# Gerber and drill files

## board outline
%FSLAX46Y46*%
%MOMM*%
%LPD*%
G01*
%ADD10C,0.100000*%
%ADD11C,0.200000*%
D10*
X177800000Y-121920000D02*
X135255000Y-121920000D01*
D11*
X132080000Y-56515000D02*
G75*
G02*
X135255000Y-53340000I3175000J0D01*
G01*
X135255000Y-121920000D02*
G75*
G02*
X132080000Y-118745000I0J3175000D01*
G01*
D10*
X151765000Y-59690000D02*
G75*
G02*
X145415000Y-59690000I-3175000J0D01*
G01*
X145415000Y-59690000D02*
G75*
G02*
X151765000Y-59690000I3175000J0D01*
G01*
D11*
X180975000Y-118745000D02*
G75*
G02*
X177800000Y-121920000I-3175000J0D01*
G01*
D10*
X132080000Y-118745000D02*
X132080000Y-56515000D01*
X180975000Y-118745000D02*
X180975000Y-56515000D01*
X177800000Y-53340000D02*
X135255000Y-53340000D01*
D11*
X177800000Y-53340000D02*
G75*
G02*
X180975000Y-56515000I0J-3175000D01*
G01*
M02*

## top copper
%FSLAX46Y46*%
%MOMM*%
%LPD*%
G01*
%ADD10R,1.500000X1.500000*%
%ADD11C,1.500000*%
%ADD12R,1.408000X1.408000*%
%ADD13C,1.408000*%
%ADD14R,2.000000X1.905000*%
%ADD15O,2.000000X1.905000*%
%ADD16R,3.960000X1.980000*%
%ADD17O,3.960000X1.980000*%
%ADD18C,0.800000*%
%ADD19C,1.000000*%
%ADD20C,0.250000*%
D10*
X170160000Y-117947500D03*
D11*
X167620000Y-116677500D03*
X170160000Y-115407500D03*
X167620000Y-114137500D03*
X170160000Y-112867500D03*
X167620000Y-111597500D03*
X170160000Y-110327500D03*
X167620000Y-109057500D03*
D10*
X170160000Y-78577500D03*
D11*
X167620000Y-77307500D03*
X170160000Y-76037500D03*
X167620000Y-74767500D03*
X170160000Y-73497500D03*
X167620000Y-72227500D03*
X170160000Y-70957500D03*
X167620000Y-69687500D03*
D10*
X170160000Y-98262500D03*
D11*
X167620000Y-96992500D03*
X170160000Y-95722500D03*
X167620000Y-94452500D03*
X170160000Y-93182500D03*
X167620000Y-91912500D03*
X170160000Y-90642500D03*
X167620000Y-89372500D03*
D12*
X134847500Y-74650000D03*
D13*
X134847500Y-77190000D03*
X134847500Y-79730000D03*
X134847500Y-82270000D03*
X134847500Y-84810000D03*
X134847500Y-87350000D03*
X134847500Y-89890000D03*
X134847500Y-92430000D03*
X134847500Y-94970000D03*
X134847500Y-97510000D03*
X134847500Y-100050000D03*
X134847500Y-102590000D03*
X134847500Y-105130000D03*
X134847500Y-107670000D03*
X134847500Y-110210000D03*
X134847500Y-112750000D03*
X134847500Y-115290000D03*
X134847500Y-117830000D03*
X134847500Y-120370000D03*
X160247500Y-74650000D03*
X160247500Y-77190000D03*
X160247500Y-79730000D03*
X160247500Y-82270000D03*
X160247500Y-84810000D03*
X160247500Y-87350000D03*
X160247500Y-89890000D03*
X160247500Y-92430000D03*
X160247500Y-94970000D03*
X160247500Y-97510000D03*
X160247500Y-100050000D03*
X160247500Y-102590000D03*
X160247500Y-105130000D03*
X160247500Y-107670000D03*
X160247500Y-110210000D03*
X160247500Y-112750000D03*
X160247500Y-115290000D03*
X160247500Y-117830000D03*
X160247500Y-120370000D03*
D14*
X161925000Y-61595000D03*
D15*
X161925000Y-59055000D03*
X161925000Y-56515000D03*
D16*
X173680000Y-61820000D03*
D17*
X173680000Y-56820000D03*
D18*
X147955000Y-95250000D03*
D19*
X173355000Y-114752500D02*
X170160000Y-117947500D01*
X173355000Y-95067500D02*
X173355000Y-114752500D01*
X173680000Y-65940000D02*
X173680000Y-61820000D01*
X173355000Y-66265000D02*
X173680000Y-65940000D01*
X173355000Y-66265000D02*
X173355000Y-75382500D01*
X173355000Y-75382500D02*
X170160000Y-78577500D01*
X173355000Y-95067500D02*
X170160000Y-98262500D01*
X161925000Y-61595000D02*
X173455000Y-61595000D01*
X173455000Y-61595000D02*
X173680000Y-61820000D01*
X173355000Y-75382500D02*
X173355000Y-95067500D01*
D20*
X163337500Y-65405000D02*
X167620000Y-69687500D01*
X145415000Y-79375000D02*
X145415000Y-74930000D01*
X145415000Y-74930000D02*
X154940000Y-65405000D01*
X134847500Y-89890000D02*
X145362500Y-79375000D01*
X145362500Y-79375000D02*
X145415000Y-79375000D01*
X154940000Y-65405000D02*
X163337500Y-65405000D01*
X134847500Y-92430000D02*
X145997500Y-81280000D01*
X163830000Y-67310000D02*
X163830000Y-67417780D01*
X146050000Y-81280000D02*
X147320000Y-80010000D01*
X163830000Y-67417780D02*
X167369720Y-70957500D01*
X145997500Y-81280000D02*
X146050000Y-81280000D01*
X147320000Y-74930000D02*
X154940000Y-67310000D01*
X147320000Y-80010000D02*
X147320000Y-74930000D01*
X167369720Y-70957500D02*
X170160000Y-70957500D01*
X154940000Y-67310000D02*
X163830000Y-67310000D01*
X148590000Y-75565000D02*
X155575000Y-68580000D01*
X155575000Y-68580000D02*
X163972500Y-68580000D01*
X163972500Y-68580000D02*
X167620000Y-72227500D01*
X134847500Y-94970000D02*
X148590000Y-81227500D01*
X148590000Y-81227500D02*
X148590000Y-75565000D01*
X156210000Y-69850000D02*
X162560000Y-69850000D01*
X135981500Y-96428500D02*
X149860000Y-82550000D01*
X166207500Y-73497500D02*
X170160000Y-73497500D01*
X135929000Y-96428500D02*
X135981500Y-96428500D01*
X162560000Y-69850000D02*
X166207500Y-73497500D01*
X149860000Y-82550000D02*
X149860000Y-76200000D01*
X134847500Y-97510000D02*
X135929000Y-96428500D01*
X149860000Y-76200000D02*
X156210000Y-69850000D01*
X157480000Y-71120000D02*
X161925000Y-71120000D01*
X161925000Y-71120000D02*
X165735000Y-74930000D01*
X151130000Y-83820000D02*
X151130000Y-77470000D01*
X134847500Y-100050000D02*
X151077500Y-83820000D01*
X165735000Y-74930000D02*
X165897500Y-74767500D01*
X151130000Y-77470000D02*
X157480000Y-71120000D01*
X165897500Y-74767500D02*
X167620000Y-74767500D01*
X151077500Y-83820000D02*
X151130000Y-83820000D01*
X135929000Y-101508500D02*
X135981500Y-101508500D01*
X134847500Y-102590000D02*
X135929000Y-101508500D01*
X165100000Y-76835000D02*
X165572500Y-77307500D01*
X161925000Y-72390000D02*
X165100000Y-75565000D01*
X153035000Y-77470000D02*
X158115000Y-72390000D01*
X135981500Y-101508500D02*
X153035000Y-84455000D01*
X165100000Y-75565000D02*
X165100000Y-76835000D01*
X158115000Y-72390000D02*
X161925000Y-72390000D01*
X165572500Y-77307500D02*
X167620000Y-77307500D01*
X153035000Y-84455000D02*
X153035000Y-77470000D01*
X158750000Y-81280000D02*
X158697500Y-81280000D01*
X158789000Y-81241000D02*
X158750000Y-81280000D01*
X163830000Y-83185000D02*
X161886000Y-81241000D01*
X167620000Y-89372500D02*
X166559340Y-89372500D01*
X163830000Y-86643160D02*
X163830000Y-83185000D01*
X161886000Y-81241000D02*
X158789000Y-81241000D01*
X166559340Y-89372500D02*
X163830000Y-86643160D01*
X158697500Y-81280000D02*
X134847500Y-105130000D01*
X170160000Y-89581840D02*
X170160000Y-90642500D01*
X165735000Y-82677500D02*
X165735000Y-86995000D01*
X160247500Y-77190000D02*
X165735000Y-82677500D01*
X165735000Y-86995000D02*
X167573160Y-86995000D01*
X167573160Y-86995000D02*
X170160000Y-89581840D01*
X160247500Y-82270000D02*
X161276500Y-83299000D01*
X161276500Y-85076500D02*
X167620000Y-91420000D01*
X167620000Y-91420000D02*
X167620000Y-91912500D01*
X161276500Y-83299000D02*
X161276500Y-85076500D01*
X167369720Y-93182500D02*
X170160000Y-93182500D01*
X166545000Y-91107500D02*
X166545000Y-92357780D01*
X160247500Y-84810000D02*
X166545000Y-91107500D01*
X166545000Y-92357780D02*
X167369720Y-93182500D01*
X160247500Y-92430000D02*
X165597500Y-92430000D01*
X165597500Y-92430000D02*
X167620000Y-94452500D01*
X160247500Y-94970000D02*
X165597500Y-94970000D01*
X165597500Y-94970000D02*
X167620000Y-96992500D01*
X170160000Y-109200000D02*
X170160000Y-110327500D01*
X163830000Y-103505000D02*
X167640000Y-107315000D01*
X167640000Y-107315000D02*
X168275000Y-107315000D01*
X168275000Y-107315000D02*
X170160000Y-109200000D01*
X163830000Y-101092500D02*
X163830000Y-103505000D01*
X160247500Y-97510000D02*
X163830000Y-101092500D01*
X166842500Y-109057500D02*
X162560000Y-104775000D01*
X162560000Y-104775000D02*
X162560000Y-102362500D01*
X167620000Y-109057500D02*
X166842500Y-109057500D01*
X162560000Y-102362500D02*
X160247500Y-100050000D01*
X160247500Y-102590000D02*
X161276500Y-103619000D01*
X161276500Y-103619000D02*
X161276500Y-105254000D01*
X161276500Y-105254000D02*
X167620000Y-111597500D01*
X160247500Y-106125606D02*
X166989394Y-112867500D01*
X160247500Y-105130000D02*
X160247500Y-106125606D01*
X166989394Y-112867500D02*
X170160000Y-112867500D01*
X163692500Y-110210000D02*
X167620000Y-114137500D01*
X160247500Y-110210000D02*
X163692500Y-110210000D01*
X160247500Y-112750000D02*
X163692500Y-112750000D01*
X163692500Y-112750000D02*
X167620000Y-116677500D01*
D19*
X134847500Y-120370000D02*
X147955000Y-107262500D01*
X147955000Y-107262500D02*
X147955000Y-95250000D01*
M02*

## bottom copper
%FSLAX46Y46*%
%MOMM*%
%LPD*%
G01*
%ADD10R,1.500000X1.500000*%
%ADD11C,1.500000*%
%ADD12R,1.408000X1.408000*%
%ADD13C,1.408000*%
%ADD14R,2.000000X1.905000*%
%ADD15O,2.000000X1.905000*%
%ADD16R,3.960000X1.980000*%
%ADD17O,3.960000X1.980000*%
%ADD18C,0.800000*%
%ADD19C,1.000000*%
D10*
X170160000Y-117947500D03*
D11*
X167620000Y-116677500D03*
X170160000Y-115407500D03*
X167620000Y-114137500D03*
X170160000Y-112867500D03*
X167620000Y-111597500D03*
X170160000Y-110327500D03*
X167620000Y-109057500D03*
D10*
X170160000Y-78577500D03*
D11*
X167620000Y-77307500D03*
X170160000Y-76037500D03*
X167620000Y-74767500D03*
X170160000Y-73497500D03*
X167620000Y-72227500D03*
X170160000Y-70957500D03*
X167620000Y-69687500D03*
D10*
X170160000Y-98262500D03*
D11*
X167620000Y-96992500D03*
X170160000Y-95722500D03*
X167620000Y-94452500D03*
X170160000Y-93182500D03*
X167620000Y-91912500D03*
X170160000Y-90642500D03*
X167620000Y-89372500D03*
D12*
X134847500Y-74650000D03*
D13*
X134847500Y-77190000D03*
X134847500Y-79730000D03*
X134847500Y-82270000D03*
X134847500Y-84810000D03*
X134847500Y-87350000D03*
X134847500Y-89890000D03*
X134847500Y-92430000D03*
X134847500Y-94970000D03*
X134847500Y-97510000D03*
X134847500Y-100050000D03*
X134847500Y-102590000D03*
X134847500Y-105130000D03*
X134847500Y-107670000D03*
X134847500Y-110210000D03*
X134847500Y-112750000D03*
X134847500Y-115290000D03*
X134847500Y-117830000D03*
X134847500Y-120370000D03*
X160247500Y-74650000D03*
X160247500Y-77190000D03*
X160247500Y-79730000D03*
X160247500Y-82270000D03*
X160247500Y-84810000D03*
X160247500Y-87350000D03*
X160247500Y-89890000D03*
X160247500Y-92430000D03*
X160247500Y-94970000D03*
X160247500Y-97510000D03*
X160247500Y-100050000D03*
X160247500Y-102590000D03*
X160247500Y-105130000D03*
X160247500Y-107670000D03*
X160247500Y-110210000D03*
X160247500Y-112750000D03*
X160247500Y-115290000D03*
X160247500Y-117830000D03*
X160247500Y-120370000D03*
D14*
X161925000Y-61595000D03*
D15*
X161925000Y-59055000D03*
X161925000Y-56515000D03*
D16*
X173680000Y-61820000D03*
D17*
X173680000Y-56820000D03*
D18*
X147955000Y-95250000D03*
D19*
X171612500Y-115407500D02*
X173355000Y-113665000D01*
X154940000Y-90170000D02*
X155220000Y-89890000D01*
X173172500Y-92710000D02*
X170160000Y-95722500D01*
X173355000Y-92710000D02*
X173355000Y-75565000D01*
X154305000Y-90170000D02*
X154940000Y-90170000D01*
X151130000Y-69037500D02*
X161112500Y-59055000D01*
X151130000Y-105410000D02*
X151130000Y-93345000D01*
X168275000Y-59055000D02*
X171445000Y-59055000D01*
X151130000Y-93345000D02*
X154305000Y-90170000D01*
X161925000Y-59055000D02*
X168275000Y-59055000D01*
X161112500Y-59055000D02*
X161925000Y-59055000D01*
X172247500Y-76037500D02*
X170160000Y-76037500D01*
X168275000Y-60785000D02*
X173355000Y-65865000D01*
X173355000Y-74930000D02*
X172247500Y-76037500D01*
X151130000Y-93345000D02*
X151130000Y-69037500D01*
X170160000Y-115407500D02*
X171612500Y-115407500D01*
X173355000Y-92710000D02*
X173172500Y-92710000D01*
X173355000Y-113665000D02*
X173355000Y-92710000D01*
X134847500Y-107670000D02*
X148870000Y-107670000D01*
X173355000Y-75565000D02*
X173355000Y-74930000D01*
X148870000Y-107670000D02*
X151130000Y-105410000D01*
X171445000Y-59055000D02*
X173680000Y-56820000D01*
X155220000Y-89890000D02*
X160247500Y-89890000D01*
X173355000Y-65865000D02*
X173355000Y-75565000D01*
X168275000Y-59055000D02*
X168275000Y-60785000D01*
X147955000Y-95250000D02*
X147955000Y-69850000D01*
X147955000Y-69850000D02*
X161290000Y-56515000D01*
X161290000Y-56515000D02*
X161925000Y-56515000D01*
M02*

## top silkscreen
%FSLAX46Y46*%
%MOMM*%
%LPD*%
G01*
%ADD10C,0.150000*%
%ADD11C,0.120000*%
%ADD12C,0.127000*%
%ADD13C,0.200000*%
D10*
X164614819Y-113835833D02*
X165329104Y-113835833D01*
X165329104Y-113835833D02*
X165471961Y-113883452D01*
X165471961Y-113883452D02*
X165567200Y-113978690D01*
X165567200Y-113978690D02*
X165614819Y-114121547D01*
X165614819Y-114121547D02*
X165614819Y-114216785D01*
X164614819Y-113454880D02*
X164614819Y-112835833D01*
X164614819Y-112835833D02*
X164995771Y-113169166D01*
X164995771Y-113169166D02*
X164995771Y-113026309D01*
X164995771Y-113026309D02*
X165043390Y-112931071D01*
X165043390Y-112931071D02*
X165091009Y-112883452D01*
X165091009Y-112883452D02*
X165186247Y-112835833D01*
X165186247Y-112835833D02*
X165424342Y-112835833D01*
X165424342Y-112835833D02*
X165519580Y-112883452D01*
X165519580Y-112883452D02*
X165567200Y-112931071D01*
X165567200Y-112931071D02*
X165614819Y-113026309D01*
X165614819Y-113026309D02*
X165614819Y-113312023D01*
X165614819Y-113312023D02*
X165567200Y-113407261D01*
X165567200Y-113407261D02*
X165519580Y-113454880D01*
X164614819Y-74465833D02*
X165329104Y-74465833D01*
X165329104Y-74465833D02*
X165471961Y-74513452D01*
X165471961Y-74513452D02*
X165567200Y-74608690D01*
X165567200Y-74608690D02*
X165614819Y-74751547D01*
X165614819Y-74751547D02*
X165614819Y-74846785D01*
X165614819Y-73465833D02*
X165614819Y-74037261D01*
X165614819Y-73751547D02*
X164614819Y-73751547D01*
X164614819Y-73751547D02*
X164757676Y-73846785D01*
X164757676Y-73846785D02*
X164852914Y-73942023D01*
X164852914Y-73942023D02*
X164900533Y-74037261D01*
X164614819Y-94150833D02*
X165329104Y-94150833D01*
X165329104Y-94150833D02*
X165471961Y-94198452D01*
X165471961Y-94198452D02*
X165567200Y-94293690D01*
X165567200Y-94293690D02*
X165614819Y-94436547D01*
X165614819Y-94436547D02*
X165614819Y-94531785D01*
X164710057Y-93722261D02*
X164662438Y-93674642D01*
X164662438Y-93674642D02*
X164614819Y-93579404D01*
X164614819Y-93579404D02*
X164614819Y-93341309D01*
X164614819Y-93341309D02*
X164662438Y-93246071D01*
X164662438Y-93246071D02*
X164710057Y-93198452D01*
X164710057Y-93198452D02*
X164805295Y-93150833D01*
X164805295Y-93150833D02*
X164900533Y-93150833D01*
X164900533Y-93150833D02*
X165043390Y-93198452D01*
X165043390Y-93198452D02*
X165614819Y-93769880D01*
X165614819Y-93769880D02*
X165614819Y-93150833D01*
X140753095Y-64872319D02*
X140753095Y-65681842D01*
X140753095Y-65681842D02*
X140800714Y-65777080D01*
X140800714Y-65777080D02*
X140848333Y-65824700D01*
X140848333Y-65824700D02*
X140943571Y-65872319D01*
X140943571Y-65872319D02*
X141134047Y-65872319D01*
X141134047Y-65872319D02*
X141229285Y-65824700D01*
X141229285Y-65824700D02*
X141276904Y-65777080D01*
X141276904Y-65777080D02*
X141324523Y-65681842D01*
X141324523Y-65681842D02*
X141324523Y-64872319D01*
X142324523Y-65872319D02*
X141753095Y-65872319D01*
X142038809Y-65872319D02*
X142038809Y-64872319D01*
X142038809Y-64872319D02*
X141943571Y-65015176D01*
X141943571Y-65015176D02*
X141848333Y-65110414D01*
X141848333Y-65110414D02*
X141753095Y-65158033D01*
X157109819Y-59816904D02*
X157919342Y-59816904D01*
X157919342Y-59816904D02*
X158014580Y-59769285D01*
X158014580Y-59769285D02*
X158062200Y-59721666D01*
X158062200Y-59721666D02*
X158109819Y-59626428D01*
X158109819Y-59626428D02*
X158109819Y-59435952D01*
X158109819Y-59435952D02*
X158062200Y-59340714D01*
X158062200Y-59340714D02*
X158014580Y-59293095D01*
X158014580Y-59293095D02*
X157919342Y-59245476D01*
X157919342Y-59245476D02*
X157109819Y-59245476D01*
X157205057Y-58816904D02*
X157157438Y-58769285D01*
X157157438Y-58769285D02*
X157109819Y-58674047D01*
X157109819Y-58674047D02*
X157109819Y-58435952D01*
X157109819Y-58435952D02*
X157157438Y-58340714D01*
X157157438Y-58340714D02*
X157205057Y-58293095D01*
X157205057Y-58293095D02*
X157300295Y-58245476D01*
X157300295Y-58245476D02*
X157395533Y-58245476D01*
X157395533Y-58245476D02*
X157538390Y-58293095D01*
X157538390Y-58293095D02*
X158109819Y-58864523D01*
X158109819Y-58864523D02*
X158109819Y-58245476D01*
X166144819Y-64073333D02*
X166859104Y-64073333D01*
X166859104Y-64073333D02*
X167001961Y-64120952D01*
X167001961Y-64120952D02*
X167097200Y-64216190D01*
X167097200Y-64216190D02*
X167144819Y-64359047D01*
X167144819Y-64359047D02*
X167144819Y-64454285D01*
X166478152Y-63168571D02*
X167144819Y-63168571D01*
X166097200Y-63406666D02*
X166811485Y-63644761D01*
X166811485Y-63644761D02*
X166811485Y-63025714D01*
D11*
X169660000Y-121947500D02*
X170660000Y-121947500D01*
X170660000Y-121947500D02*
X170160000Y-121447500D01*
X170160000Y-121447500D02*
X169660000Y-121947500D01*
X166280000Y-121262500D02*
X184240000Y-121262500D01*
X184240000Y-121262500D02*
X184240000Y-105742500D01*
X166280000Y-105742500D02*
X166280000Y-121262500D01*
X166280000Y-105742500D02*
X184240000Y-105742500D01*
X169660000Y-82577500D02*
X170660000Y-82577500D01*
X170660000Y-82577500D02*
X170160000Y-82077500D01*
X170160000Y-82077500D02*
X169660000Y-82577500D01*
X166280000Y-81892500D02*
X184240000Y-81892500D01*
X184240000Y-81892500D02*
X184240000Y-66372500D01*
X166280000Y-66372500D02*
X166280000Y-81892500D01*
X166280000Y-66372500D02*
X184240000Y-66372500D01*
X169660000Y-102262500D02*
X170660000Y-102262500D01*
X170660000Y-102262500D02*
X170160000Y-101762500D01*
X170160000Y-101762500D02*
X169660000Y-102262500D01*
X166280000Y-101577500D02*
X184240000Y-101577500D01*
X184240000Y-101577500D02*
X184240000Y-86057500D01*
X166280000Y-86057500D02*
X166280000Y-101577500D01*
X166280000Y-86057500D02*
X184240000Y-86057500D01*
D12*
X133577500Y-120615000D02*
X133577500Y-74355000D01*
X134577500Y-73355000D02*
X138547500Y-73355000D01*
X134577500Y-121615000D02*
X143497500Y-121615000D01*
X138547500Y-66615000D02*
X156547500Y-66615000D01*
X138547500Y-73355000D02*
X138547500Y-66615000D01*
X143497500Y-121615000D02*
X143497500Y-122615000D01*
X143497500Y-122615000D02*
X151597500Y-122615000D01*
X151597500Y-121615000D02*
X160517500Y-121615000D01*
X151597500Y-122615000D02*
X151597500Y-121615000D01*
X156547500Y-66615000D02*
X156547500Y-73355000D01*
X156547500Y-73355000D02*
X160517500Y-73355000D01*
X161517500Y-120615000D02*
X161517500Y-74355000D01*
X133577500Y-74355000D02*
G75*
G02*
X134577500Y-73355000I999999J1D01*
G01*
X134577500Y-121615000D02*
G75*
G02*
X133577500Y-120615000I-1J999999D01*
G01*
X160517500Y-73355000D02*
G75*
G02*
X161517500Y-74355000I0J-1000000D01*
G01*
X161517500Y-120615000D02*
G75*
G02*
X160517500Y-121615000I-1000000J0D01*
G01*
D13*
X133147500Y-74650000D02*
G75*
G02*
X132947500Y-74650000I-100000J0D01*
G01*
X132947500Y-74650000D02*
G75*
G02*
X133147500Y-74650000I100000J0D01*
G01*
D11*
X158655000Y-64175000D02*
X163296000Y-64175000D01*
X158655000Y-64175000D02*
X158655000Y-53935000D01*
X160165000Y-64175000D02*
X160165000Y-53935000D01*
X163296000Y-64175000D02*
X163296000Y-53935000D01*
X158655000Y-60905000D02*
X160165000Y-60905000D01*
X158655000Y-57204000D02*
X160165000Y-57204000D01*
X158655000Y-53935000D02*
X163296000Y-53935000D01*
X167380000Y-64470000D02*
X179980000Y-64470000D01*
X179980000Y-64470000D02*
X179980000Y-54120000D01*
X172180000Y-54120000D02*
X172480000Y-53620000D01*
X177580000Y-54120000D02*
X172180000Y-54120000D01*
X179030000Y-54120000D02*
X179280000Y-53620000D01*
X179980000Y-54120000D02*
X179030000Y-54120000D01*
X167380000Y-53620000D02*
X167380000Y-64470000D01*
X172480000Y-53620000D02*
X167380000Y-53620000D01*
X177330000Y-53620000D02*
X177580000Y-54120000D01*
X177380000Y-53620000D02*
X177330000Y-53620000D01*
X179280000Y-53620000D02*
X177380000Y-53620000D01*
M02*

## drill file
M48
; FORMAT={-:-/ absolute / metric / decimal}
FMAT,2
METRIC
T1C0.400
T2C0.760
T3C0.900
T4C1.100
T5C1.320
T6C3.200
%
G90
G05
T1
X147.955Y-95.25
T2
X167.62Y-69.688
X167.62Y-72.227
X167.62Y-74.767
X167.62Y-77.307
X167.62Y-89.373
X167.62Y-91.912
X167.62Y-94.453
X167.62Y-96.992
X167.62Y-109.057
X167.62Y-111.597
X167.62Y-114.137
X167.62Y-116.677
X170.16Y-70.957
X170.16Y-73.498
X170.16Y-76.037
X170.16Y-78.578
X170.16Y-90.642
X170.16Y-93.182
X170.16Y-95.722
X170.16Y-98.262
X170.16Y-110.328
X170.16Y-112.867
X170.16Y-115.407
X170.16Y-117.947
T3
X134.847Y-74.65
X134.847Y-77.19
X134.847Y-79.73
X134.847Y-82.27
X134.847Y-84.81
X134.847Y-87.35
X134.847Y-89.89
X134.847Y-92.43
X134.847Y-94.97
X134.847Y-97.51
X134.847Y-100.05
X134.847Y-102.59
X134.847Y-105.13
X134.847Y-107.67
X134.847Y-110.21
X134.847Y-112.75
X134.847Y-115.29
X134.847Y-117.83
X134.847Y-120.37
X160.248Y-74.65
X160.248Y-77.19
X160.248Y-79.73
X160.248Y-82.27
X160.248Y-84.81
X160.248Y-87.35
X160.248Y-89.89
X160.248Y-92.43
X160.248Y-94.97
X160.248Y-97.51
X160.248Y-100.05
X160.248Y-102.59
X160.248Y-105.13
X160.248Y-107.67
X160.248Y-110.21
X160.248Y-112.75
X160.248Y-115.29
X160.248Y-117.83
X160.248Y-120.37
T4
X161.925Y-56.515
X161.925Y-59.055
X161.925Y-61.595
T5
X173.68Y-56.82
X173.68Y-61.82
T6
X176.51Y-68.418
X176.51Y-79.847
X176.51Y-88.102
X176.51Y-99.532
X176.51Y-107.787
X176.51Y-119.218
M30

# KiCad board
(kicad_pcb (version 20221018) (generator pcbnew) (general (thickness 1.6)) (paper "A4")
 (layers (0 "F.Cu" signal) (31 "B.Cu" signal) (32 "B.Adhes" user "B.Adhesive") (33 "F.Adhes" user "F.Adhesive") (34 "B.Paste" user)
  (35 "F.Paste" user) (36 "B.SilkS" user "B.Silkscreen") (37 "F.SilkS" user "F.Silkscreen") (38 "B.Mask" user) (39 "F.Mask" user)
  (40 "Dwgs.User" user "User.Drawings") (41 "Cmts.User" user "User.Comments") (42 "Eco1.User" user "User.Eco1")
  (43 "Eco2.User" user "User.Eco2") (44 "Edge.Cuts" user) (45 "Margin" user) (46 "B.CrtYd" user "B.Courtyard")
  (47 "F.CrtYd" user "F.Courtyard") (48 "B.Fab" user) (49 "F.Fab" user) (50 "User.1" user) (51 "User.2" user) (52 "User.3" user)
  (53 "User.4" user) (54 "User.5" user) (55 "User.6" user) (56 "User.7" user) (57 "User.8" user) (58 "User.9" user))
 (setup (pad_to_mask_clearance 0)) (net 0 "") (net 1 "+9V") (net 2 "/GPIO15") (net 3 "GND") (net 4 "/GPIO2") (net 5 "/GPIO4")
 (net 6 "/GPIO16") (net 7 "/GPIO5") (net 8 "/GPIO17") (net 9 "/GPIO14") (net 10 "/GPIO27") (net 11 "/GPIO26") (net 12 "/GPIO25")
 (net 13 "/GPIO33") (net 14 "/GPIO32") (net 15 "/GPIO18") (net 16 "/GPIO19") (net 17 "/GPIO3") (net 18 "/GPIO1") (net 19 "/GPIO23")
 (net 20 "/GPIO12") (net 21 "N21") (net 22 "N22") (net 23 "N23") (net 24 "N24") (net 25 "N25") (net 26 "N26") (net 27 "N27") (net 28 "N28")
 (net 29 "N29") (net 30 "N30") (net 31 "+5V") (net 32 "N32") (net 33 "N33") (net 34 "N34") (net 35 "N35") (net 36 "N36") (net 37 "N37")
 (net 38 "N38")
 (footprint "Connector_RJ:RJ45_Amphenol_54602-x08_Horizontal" (layer "F.Cu") (at 170.16 117.9475 90)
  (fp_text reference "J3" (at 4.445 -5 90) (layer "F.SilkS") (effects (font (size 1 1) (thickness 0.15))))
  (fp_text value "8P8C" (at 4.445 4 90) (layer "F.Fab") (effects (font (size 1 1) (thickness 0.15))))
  (fp_line (start -4 -0.5) (end -4 0.5) (stroke (width 0.12) (type solid)) (layer "F.SilkS"))
  (fp_line (start -4 0.5) (end -3.5 0) (stroke (width 0.12) (type solid)) (layer "F.SilkS"))
  (fp_line (start -3.5 0) (end -4 -0.5) (stroke (width 0.12) (type solid)) (layer "F.SilkS"))
  (fp_line (start -3.315 -3.88) (end -3.315 14.08) (stroke (width 0.12) (type solid)) (layer "F.SilkS"))
  (fp_line (start -3.315 14.08) (end 12.205 14.08) (stroke (width 0.12) (type solid)) (layer "F.SilkS"))
  (fp_line (start 12.205 -3.88) (end -3.315 -3.88) (stroke (width 0.12) (type solid)) (layer "F.SilkS"))
  (fp_line (start 12.205 -3.88) (end 12.205 14.08) (stroke (width 0.12) (type solid)) (layer "F.SilkS"))
  (pad "" np_thru_hole circle (at -1.27 6.35 90) (size 3.2 3.2) (drill 3.2) (layers "*.Cu" "*.Mask"))
  (pad "" np_thru_hole circle (at 10.16 6.35 90) (size 3.2 3.2) (drill 3.2) (layers "*.Cu" "*.Mask"))
  (pad "1" thru_hole rect (at 0 0 90) (size 1.5 1.5) (drill 0.76) (layers "*.Cu" "*.Mask") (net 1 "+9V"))
  (pad "2" thru_hole circle (at 1.27 -2.54 90) (size 1.5 1.5) (drill 0.76) (layers "*.Cu" "*.Mask") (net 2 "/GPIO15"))
  (pad "3" thru_hole circle (at 2.54 0 90) (size 1.5 1.5) (drill 0.76) (layers "*.Cu" "*.Mask") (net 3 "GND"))
  (pad "4" thru_hole circle (at 3.81 -2.54 90) (size 1.5 1.5) (drill 0.76) (layers "*.Cu" "*.Mask") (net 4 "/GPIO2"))
  (pad "5" thru_hole circle (at 5.08 0 90) (size 1.5 1.5) (drill 0.76) (layers "*.Cu" "*.Mask") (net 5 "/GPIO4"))
  (pad "6" thru_hole circle (at 6.35 -2.54 90) (size 1.5 1.5) (drill 0.76) (layers "*.Cu" "*.Mask") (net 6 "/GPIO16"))
  (pad "7" thru_hole circle (at 7.62 0 90) (size 1.5 1.5) (drill 0.76) (layers "*.Cu" "*.Mask") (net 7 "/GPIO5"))
  (pad "8" thru_hole circle (at 8.89 -2.54 90) (size 1.5 1.5) (drill 0.76) (layers "*.Cu" "*.Mask") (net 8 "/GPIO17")))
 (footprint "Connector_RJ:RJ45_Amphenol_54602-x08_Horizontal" (layer "F.Cu") (at 170.16 78.5775 90)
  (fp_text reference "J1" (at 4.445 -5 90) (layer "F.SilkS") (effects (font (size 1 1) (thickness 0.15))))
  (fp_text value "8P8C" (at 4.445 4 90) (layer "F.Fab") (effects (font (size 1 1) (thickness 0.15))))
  (fp_line (start -4 -0.5) (end -4 0.5) (stroke (width 0.12) (type solid)) (layer "F.SilkS"))
  (fp_line (start -4 0.5) (end -3.5 0) (stroke (width 0.12) (type solid)) (layer "F.SilkS"))
  (fp_line (start -3.5 0) (end -4 -0.5) (stroke (width 0.12) (type solid)) (layer "F.SilkS"))
  (fp_line (start -3.315 -3.88) (end -3.315 14.08) (stroke (width 0.12) (type solid)) (layer "F.SilkS"))
  (fp_line (start -3.315 14.08) (end 12.205 14.08) (stroke (width 0.12) (type solid)) (layer "F.SilkS"))
  (fp_line (start 12.205 -3.88) (end -3.315 -3.88) (stroke (width 0.12) (type solid)) (layer "F.SilkS"))
  (fp_line (start 12.205 -3.88) (end 12.205 14.08) (stroke (width 0.12) (type solid)) (layer "F.SilkS"))
  (pad "" np_thru_hole circle (at -1.27 6.35 90) (size 3.2 3.2) (drill 3.2) (layers "*.Cu" "*.Mask"))
  (pad "" np_thru_hole circle (at 10.16 6.35 90) (size 3.2 3.2) (drill 3.2) (layers "*.Cu" "*.Mask"))
  (pad "1" thru_hole rect (at 0 0 90) (size 1.5 1.5) (drill 0.76) (layers "*.Cu" "*.Mask") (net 1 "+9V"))
  (pad "2" thru_hole circle (at 1.27 -2.54 90) (size 1.5 1.5) (drill 0.76) (layers "*.Cu" "*.Mask") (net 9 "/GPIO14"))
  (pad "3" thru_hole circle (at 2.54 0 90) (size 1.5 1.5) (drill 0.76) (layers "*.Cu" "*.Mask") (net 3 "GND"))
  (pad "4" thru_hole circle (at 3.81 -2.54 90) (size 1.5 1.5) (drill 0.76) (layers "*.Cu" "*.Mask") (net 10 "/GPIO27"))
  (pad "5" thru_hole circle (at 5.08 0 90) (size 1.5 1.5) (drill 0.76) (layers "*.Cu" "*.Mask") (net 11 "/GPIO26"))
  (pad "6" thru_hole circle (at 6.35 -2.54 90) (size 1.5 1.5) (drill 0.76) (layers "*.Cu" "*.Mask") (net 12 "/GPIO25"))
  (pad "7" thru_hole circle (at 7.62 0 90) (size 1.5 1.5) (drill 0.76) (layers "*.Cu" "*.Mask") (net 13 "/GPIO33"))
  (pad "8" thru_hole circle (at 8.89 -2.54 90) (size 1.5 1.5) (drill 0.76) (layers "*.Cu" "*.Mask") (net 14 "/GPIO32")))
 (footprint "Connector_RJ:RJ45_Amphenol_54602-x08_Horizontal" (layer "F.Cu") (at 170.16 98.2625 90)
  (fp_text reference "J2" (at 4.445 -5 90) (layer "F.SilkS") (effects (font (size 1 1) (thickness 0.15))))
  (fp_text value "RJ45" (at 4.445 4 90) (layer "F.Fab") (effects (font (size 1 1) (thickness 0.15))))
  (fp_line (start -4 -0.5) (end -4 0.5) (stroke (width 0.12) (type solid)) (layer "F.SilkS"))
  (fp_line (start -4 0.5) (end -3.5 0) (stroke (width 0.12) (type solid)) (layer "F.SilkS"))
  (fp_line (start -3.5 0) (end -4 -0.5) (stroke (width 0.12) (type solid)) (layer "F.SilkS"))
  (fp_line (start -3.315 -3.88) (end -3.315 14.08) (stroke (width 0.12) (type solid)) (layer "F.SilkS"))
  (fp_line (start -3.315 14.08) (end 12.205 14.08) (stroke (width 0.12) (type solid)) (layer "F.SilkS"))
  (fp_line (start 12.205 -3.88) (end -3.315 -3.88) (stroke (width 0.12) (type solid)) (layer "F.SilkS"))
  (fp_line (start 12.205 -3.88) (end 12.205 14.08) (stroke (width 0.12) (type solid)) (layer "F.SilkS"))
  (pad "" np_thru_hole circle (at -1.27 6.35 90) (size 3.2 3.2) (drill 3.2) (layers "*.Cu" "*.Mask"))
  (pad "" np_thru_hole circle (at 10.16 6.35 90) (size 3.2 3.2) (drill 3.2) (layers "*.Cu" "*.Mask"))
  (pad "1" thru_hole rect (at 0 0 90) (size 1.5 1.5) (drill 0.76) (layers "*.Cu" "*.Mask") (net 1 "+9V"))
  (pad "2" thru_hole circle (at 1.27 -2.54 90) (size 1.5 1.5) (drill 0.76) (layers "*.Cu" "*.Mask") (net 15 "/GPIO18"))
  (pad "3" thru_hole circle (at 2.54 0 90) (size 1.5 1.5) (drill 0.76) (layers "*.Cu" "*.Mask") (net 3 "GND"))
  (pad "4" thru_hole circle (at 3.81 -2.54 90) (size 1.5 1.5) (drill 0.76) (layers "*.Cu" "*.Mask") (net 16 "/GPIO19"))
  (pad "5" thru_hole circle (at 5.08 0 90) (size 1.5 1.5) (drill 0.76) (layers "*.Cu" "*.Mask") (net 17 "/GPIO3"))
  (pad "6" thru_hole circle (at 6.35 -2.54 90) (size 1.5 1.5) (drill 0.76) (layers "*.Cu" "*.Mask") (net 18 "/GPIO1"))
  (pad "7" thru_hole circle (at 7.62 0 90) (size 1.5 1.5) (drill 0.76) (layers "*.Cu" "*.Mask") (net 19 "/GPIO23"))
  (pad "8" thru_hole circle (at 8.89 -2.54 90) (size 1.5 1.5) (drill 0.76) (layers "*.Cu" "*.Mask") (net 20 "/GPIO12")))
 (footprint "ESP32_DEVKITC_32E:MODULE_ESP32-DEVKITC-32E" (layer "F.Cu") (at 147.5475 97.485)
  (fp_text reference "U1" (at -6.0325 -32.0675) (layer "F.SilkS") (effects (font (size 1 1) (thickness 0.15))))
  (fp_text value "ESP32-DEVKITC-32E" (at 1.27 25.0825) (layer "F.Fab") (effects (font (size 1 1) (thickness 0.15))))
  (fp_line (start -13.97 23.13) (end -13.97 -23.13) (stroke (width 0.127) (type solid)) (layer "F.SilkS"))
  (fp_line (start -12.97 -24.13) (end -9 -24.13) (stroke (width 0.127) (type solid)) (layer "F.SilkS"))
  (fp_line (start -12.97 24.13) (end -4.05 24.13) (stroke (width 0.127) (type solid)) (layer "F.SilkS"))
  (fp_line (start -9 -30.87) (end 9 -30.87) (stroke (width 0.127) (type solid)) (layer "F.SilkS"))
  (fp_line (start -9 -24.13) (end -9 -30.87) (stroke (width 0.127) (type solid)) (layer "F.SilkS"))
  (fp_line (start -4.05 24.13) (end -4.05 25.13) (stroke (width 0.127) (type solid)) (layer "F.SilkS"))
  (fp_line (start -4.05 25.13) (end 4.05 25.13) (stroke (width 0.127) (type solid)) (layer "F.SilkS"))
  (fp_line (start 4.05 24.13) (end 12.97 24.13) (stroke (width 0.127) (type solid)) (layer "F.SilkS"))
  (fp_line (start 4.05 25.13) (end 4.05 24.13) (stroke (width 0.127) (type solid)) (layer "F.SilkS"))
  (fp_line (start 9 -30.87) (end 9 -24.13) (stroke (width 0.127) (type solid)) (layer "F.SilkS"))
  (fp_line (start 9 -24.13) (end 12.97 -24.13) (stroke (width 0.127) (type solid)) (layer "F.SilkS"))
  (fp_line (start 13.97 23.13) (end 13.97 -23.13) (stroke (width 0.127) (type solid)) (layer "F.SilkS"))
  (fp_arc (start -13.97 -23.13) (mid -13.677107 -23.837107) (end -12.97 -24.13) (stroke (width 0.127) (type solid)) (layer "F.SilkS"))
  (fp_arc (start -12.97 24.13) (mid -13.677107 23.837107) (end -13.97 23.13) (stroke (width 0.127) (type solid)) (layer "F.SilkS"))
  (fp_arc (start 12.97 -24.13) (mid 13.677107 -23.837107) (end 13.97 -23.13) (stroke (width 0.127) (type solid)) (layer "F.SilkS"))
  (fp_arc (start 13.97 23.13) (mid 13.677107 23.837107) (end 12.97 24.13) (stroke (width 0.127) (type solid)) (layer "F.SilkS"))
  (fp_circle (center -14.5 -22.835) (end -14.4 -22.835) (stroke (width 0.2) (type solid)) (fill none) (layer "F.SilkS"))
  (pad "J2_1" thru_hole rect (at -12.7 -22.835) (size 1.408 1.408) (drill 0.9) (layers "*.Cu" "*.Mask") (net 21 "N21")
   (solder_mask_margin 0.102))
  (pad "J2_2" thru_hole circle (at -12.7 -20.295) (size 1.408 1.408) (drill 0.9) (layers "*.Cu" "*.Mask") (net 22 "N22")
   (solder_mask_margin 0.102))
  (pad "J2_3" thru_hole circle (at -12.7 -17.755) (size 1.408 1.408) (drill 0.9) (layers "*.Cu" "*.Mask") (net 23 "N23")
   (solder_mask_margin 0.102))
  (pad "J2_4" thru_hole circle (at -12.7 -15.215) (size 1.408 1.408) (drill 0.9) (layers "*.Cu" "*.Mask") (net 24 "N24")
   (solder_mask_margin 0.102))
  (pad "J2_5" thru_hole circle (at -12.7 -12.675) (size 1.408 1.408) (drill 0.9) (layers "*.Cu" "*.Mask") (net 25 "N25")
   (solder_mask_margin 0.102))
  (pad "J2_6" thru_hole circle (at -12.7 -10.135) (size 1.408 1.408) (drill 0.9) (layers "*.Cu" "*.Mask") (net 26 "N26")
   (solder_mask_margin 0.102))
  (pad "J2_7" thru_hole circle (at -12.7 -7.595) (size 1.408 1.408) (drill 0.9) (layers "*.Cu" "*.Mask") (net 14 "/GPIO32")
   (solder_mask_margin 0.102))
  (pad "J2_8" thru_hole circle (at -12.7 -5.055) (size 1.408 1.408) (drill 0.9) (layers "*.Cu" "*.Mask") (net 13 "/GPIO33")
   (solder_mask_margin 0.102))
  (pad "J2_9" thru_hole circle (at -12.7 -2.515) (size 1.408 1.408) (drill 0.9) (layers "*.Cu" "*.Mask") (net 12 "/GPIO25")
   (solder_mask_margin 0.102))
  (pad "J2_10" thru_hole circle (at -12.7 0.025) (size 1.408 1.408) (drill 0.9) (layers "*.Cu" "*.Mask") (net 11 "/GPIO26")
   (solder_mask_margin 0.102))
  (pad "J2_11" thru_hole circle (at -12.7 2.565) (size 1.408 1.408) (drill 0.9) (layers "*.Cu" "*.Mask") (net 10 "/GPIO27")
   (solder_mask_margin 0.102))
  (pad "J2_12" thru_hole circle (at -12.7 5.105) (size 1.408 1.408) (drill 0.9) (layers "*.Cu" "*.Mask") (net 9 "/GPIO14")
   (solder_mask_margin 0.102))
  (pad "J2_13" thru_hole circle (at -12.7 7.645) (size 1.408 1.408) (drill 0.9) (layers "*.Cu" "*.Mask") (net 20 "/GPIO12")
   (solder_mask_margin 0.102))
  (pad "J2_14" thru_hole circle (at -12.7 10.185) (size 1.408 1.408) (drill 0.9) (layers "*.Cu" "*.Mask") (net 3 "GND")
   (solder_mask_margin 0.102))
  (pad "J2_15" thru_hole circle (at -12.7 12.725) (size 1.408 1.408) (drill 0.9) (layers "*.Cu" "*.Mask") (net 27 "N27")
   (solder_mask_margin 0.102))
  (pad "J2_16" thru_hole circle (at -12.7 15.265) (size 1.408 1.408) (drill 0.9) (layers "*.Cu" "*.Mask") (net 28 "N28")
   (solder_mask_margin 0.102))
  (pad "J2_17" thru_hole circle (at -12.7 17.805) (size 1.408 1.408) (drill 0.9) (layers "*.Cu" "*.Mask") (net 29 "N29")
   (solder_mask_margin 0.102))
  (pad "J2_18" thru_hole circle (at -12.7 20.345) (size 1.408 1.408) (drill 0.9) (layers "*.Cu" "*.Mask") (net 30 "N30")
   (solder_mask_margin 0.102))
  (pad "J2_19" thru_hole circle (at -12.7 22.885) (size 1.408 1.408) (drill 0.9) (layers "*.Cu" "*.Mask") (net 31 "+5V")
   (solder_mask_margin 0.102))
  (pad "J3_1" thru_hole circle (at 12.7 -22.835) (size 1.408 1.408) (drill 0.9) (layers "*.Cu" "*.Mask") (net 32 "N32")
   (solder_mask_margin 0.102))
  (pad "J3_2" thru_hole circle (at 12.7 -20.295) (size 1.408 1.408) (drill 0.9) (layers "*.Cu" "*.Mask") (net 19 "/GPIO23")
   (solder_mask_margin 0.102))
  (pad "J3_3" thru_hole circle (at 12.7 -17.755) (size 1.408 1.408) (drill 0.9) (layers "*.Cu" "*.Mask") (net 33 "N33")
   (solder_mask_margin 0.102))
  (pad "J3_4" thru_hole circle (at 12.7 -15.215) (size 1.408 1.408) (drill 0.9) (layers "*.Cu" "*.Mask") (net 18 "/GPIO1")
   (solder_mask_margin 0.102))
  (pad "J3_5" thru_hole circle (at 12.7 -12.675) (size 1.408 1.408) (drill 0.9) (layers "*.Cu" "*.Mask") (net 17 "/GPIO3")
   (solder_mask_margin 0.102))
  (pad "J3_6" thru_hole circle (at 12.7 -10.135) (size 1.408 1.408) (drill 0.9) (layers "*.Cu" "*.Mask") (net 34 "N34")
   (solder_mask_margin 0.102))
  (pad "J3_7" thru_hole circle (at 12.7 -7.595) (size 1.408 1.408) (drill 0.9) (layers "*.Cu" "*.Mask") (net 3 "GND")
   (solder_mask_margin 0.102))
  (pad "J3_8" thru_hole circle (at 12.7 -5.055) (size 1.408 1.408) (drill 0.9) (layers "*.Cu" "*.Mask") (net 16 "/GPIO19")
   (solder_mask_margin 0.102))
  (pad "J3_9" thru_hole circle (at 12.7 -2.515) (size 1.408 1.408) (drill 0.9) (layers "*.Cu" "*.Mask") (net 15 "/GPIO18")
   (solder_mask_margin 0.102))
  (pad "J3_10" thru_hole circle (at 12.7 0.025) (size 1.408 1.408) (drill 0.9) (layers "*.Cu" "*.Mask") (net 7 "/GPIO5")
   (solder_mask_margin 0.102))
  (pad "J3_11" thru_hole circle (at 12.7 2.565) (size 1.408 1.408) (drill 0.9) (layers "*.Cu" "*.Mask") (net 8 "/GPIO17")
   (solder_mask_margin 0.102))
  (pad "J3_12" thru_hole circle (at 12.7 5.105) (size 1.408 1.408) (drill 0.9) (layers "*.Cu" "*.Mask") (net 6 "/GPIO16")
   (solder_mask_margin 0.102))
  (pad "J3_13" thru_hole circle (at 12.7 7.645) (size 1.408 1.408) (drill 0.9) (layers "*.Cu" "*.Mask") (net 5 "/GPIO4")
   (solder_mask_margin 0.102))
  (pad "J3_14" thru_hole circle (at 12.7 10.185) (size 1.408 1.408) (drill 0.9) (layers "*.Cu" "*.Mask") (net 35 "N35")
   (solder_mask_margin 0.102))
  (pad "J3_15" thru_hole circle (at 12.7 12.725) (size 1.408 1.408) (drill 0.9) (layers "*.Cu" "*.Mask") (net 4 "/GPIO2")
   (solder_mask_margin 0.102))
  (pad "J3_16" thru_hole circle (at 12.7 15.265) (size 1.408 1.408) (drill 0.9) (layers "*.Cu" "*.Mask") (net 2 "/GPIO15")
   (solder_mask_margin 0.102))
  (pad "J3_17" thru_hole circle (at 12.7 17.805) (size 1.408 1.408) (drill 0.9) (layers "*.Cu" "*.Mask") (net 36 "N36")
   (solder_mask_margin 0.102))
  (pad "J3_18" thru_hole circle (at 12.7 20.345) (size 1.408 1.408) (drill 0.9) (layers "*.Cu" "*.Mask") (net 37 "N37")
   (solder_mask_margin 0.102))
  (pad "J3_19" thru_hole circle (at 12.7 22.885) (size 1.408 1.408) (drill 0.9) (layers "*.Cu" "*.Mask") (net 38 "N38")
   (solder_mask_margin 0.102)))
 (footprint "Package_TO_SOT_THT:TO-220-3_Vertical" (layer "F.Cu") (at 161.925 61.595 90)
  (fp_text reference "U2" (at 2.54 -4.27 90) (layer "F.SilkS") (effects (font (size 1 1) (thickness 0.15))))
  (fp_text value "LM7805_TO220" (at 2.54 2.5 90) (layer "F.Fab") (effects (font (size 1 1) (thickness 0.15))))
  (fp_line (start -2.58 -3.27) (end -2.58 1.371) (stroke (width 0.12) (type solid)) (layer "F.SilkS"))
  (fp_line (start -2.58 -3.27) (end 7.66 -3.27) (stroke (width 0.12) (type solid)) (layer "F.SilkS"))
  (fp_line (start -2.58 -1.76) (end 7.66 -1.76) (stroke (width 0.12) (type solid)) (layer "F.SilkS"))
  (fp_line (start -2.58 1.371) (end 7.66 1.371) (stroke (width 0.12) (type solid)) (layer "F.SilkS"))
  (fp_line (start 0.69 -3.27) (end 0.69 -1.76) (stroke (width 0.12) (type solid)) (layer "F.SilkS"))
  (fp_line (start 4.391 -3.27) (end 4.391 -1.76) (stroke (width 0.12) (type solid)) (layer "F.SilkS"))
  (fp_line (start 7.66 -3.27) (end 7.66 1.371) (stroke (width 0.12) (type solid)) (layer "F.SilkS"))
  (pad "1" thru_hole rect (at 0 0 90) (size 1.905 2) (drill 1.1) (layers "*.Cu" "*.Mask") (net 1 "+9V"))
  (pad "2" thru_hole oval (at 2.54 0 90) (size 1.905 2) (drill 1.1) (layers "*.Cu" "*.Mask") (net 3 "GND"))
  (pad "3" thru_hole oval (at 5.08 0 90) (size 1.905 2) (drill 1.1) (layers "*.Cu" "*.Mask") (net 31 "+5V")))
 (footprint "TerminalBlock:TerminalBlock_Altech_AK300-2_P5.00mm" (layer "F.Cu") (at 173.68 61.82 90)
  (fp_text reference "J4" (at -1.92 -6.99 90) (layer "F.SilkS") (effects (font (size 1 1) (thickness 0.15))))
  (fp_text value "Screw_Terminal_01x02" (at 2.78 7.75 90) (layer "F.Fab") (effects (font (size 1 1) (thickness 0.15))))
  (fp_line (start -2.65 -6.3) (end -2.65 6.3) (stroke (width 0.12) (type solid)) (layer "F.SilkS"))
  (fp_line (start -2.65 6.3) (end 7.7 6.3) (stroke (width 0.12) (type solid)) (layer "F.SilkS"))
  (fp_line (start 7.7 -1.5) (end 8.2 -1.2) (stroke (width 0.12) (type solid)) (layer "F.SilkS"))
  (fp_line (start 7.7 3.9) (end 7.7 -1.5) (stroke (width 0.12) (type solid)) (layer "F.SilkS"))
  (fp_line (start 7.7 5.35) (end 8.2 5.6) (stroke (width 0.12) (type solid)) (layer "F.SilkS"))
  (fp_line (start 7.7 6.3) (end 7.7 5.35) (stroke (width 0.12) (type solid)) (layer "F.SilkS"))
  (fp_line (start 8.2 -6.3) (end -2.65 -6.3) (stroke (width 0.12) (type solid)) (layer "F.SilkS"))
  (fp_line (start 8.2 -1.2) (end 8.2 -6.3) (stroke (width 0.12) (type solid)) (layer "F.SilkS"))
  (fp_line (start 8.2 3.65) (end 7.7 3.9) (stroke (width 0.12) (type solid)) (layer "F.SilkS"))
  (fp_line (start 8.2 3.7) (end 8.2 3.65) (stroke (width 0.12) (type solid)) (layer "F.SilkS"))
  (fp_line (start 8.2 5.6) (end 8.2 3.7) (stroke (width 0.12) (type solid)) (layer "F.SilkS"))
  (pad "1" thru_hole rect (at 0 0 90) (size 1.98 3.96) (drill 1.32) (layers "*.Cu" "*.Mask") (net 1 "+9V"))
  (pad "2" thru_hole oval (at 5 0 90) (size 1.98 3.96) (drill 1.32) (layers "*.Cu" "*.Mask") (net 3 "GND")))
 (gr_line (start 177.8 121.92) (end 135.255 121.92) (stroke (width 0.1) (type default)) (layer "Edge.Cuts"))
 (gr_arc (start 132.08 56.515) (mid 133.009936 54.269936) (end 135.255 53.34) (stroke (width 0.2) (type default)) (layer "Edge.Cuts"))
 (gr_arc (start 135.255 121.92) (mid 133.009936 120.990064) (end 132.08 118.745) (stroke (width 0.2) (type default)) (layer "Edge.Cuts"))
 (gr_circle (center 148.59 59.69) (end 145.415 59.69) (stroke (width 0.1) (type default)) (fill none) (layer "Edge.Cuts"))
 (gr_arc (start 180.975 118.745) (mid 180.045064 120.990064) (end 177.8 121.92) (stroke (width 0.2) (type default)) (layer "Edge.Cuts"))
 (gr_line (start 132.08 118.745) (end 132.08 56.515) (stroke (width 0.1) (type default)) (layer "Edge.Cuts"))
 (gr_line (start 180.975 118.745) (end 180.975 56.515) (stroke (width 0.1) (type default)) (layer "Edge.Cuts"))
 (gr_line (start 177.8 53.34) (end 135.255 53.34) (stroke (width 0.1) (type default)) (layer "Edge.Cuts"))
 (gr_arc (start 177.8 53.34) (mid 180.045064 54.269936) (end 180.975 56.515) (stroke (width 0.2) (type default)) (layer "Edge.Cuts"))
 (segment (start 173.355 114.7525) (end 170.16 117.9475) (width 1) (layer "F.Cu") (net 1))
 (segment (start 173.355 95.0675) (end 173.355 114.7525) (width 1) (layer "F.Cu") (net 1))
 (segment (start 173.68 65.94) (end 173.68 61.82) (width 1) (layer "F.Cu") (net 1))
 (segment (start 173.355 66.265) (end 173.68 65.94) (width 1) (layer "F.Cu") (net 1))
 (segment (start 173.355 66.265) (end 173.355 75.3825) (width 1) (layer "F.Cu") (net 1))
 (segment (start 173.355 75.3825) (end 170.16 78.5775) (width 1) (layer "F.Cu") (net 1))
 (segment (start 173.355 95.0675) (end 170.16 98.2625) (width 1) (layer "F.Cu") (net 1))
 (segment (start 161.925 61.595) (end 173.455 61.595) (width 1) (layer "F.Cu") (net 1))
 (segment (start 173.455 61.595) (end 173.68 61.82) (width 1) (layer "F.Cu") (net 1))
 (segment (start 173.355 75.3825) (end 173.355 95.0675) (width 1) (layer "F.Cu") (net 1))
 (segment (start 171.6125 115.4075) (end 173.355 113.665) (width 1) (layer "B.Cu") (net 3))
 (segment (start 154.94 90.17) (end 155.22 89.89) (width 1) (layer "B.Cu") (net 3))
 (segment (start 173.1725 92.71) (end 170.16 95.7225) (width 1) (layer "B.Cu") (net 3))
 (segment (start 173.355 92.71) (end 173.355 75.565) (width 1) (layer "B.Cu") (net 3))
 (segment (start 154.305 90.17) (end 154.94 90.17) (width 1) (layer "B.Cu") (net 3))
 (segment (start 151.13 69.0375) (end 161.1125 59.055) (width 1) (layer "B.Cu") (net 3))
 (segment (start 151.13 105.41) (end 151.13 93.345) (width 1) (layer "B.Cu") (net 3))
 (segment (start 168.275 59.055) (end 171.445 59.055) (width 1) (layer "B.Cu") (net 3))
 (segment (start 151.13 93.345) (end 154.305 90.17) (width 1) (layer "B.Cu") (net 3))
 (segment (start 161.925 59.055) (end 168.275 59.055) (width 1) (layer "B.Cu") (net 3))
 (segment (start 161.1125 59.055) (end 161.925 59.055) (width 1) (layer "B.Cu") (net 3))
 (segment (start 172.2475 76.0375) (end 170.16 76.0375) (width 1) (layer "B.Cu") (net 3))
 (segment (start 168.275 60.785) (end 173.355 65.865) (width 1) (layer "B.Cu") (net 3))
 (segment (start 173.355 74.93) (end 172.2475 76.0375) (width 1) (layer "B.Cu") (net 3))
 (segment (start 151.13 93.345) (end 151.13 69.0375) (width 1) (layer "B.Cu") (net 3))
 (segment (start 170.16 115.4075) (end 171.6125 115.4075) (width 1) (layer "B.Cu") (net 3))
 (segment (start 173.355 92.71) (end 173.1725 92.71) (width 1) (layer "B.Cu") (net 3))
 (segment (start 173.355 113.665) (end 173.355 92.71) (width 1) (layer "B.Cu") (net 3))
 (segment (start 134.8475 107.67) (end 148.87 107.67) (width 1) (layer "B.Cu") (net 3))
 (segment (start 173.355 75.565) (end 173.355 74.93) (width 1) (layer "B.Cu") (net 3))
 (segment (start 148.87 107.67) (end 151.13 105.41) (width 1) (layer "B.Cu") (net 3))
 (segment (start 171.445 59.055) (end 173.68 56.82) (width 1) (layer "B.Cu") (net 3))
 (segment (start 155.22 89.89) (end 160.2475 89.89) (width 1) (layer "B.Cu") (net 3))
 (segment (start 173.355 65.865) (end 173.355 75.565) (width 1) (layer "B.Cu") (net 3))
 (segment (start 168.275 59.055) (end 168.275 60.785) (width 1) (layer "B.Cu") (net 3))
 (segment (start 163.3375 65.405) (end 167.62 69.6875) (width 0.25) (layer "F.Cu") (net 14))
 (segment (start 145.415 79.375) (end 145.415 74.93) (width 0.25) (layer "F.Cu") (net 14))
 (segment (start 145.415 74.93) (end 154.94 65.405) (width 0.25) (layer "F.Cu") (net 14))
 (segment (start 134.8475 89.89) (end 145.3625 79.375) (width 0.25) (layer "F.Cu") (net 14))
 (segment (start 145.3625 79.375) (end 145.415 79.375) (width 0.25) (layer "F.Cu") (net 14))
 (segment (start 154.94 65.405) (end 163.3375 65.405) (width 0.25) (layer "F.Cu") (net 14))
 (segment (start 134.8475 92.43) (end 145.9975 81.28) (width 0.25) (layer "F.Cu") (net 13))
 (segment (start 163.83 67.31) (end 163.83 67.41778) (width 0.25) (layer "F.Cu") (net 13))
 (segment (start 146.05 81.28) (end 147.32 80.01) (width 0.25) (layer "F.Cu") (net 13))
 (segment (start 163.83 67.41778) (end 167.36972 70.9575) (width 0.25) (layer "F.Cu") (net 13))
 (segment (start 145.9975 81.28) (end 146.05 81.28) (width 0.25) (layer "F.Cu") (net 13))
 (segment (start 147.32 74.93) (end 154.94 67.31) (width 0.25) (layer "F.Cu") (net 13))
 (segment (start 147.32 80.01) (end 147.32 74.93) (width 0.25) (layer "F.Cu") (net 13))
 (segment (start 167.36972 70.9575) (end 170.16 70.9575) (width 0.25) (layer "F.Cu") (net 13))
 (segment (start 154.94 67.31) (end 163.83 67.31) (width 0.25) (layer "F.Cu") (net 13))
 (segment (start 148.59 75.565) (end 155.575 68.58) (width 0.25) (layer "F.Cu") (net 12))
 (segment (start 155.575 68.58) (end 163.9725 68.58) (width 0.25) (layer "F.Cu") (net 12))
 (segment (start 163.9725 68.58) (end 167.62 72.2275) (width 0.25) (layer "F.Cu") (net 12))
 (segment (start 134.8475 94.97) (end 148.59 81.2275) (width 0.25) (layer "F.Cu") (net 12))
 (segment (start 148.59 81.2275) (end 148.59 75.565) (width 0.25) (layer "F.Cu") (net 12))
 (segment (start 156.21 69.85) (end 162.56 69.85) (width 0.25) (layer "F.Cu") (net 11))
 (segment (start 135.9815 96.4285) (end 149.86 82.55) (width 0.25) (layer "F.Cu") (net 11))
 (segment (start 166.2075 73.4975) (end 170.16 73.4975) (width 0.25) (layer "F.Cu") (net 11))
 (segment (start 135.929 96.4285) (end 135.9815 96.4285) (width 0.25) (layer "F.Cu") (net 11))
 (segment (start 162.56 69.85) (end 166.2075 73.4975) (width 0.25) (layer "F.Cu") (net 11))
 (segment (start 149.86 82.55) (end 149.86 76.2) (width 0.25) (layer "F.Cu") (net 11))
 (segment (start 134.8475 97.51) (end 135.929 96.4285) (width 0.25) (layer "F.Cu") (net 11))
 (segment (start 149.86 76.2) (end 156.21 69.85) (width 0.25) (layer "F.Cu") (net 11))
 (segment (start 157.48 71.12) (end 161.925 71.12) (width 0.25) (layer "F.Cu") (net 10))
 (segment (start 161.925 71.12) (end 165.735 74.93) (width 0.25) (layer "F.Cu") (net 10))
 (segment (start 151.13 83.82) (end 151.13 77.47) (width 0.25) (layer "F.Cu") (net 10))
 (segment (start 134.8475 100.05) (end 151.0775 83.82) (width 0.25) (layer "F.Cu") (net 10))
 (segment (start 165.735 74.93) (end 165.8975 74.7675) (width 0.25) (layer "F.Cu") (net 10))
 (segment (start 151.13 77.47) (end 157.48 71.12) (width 0.25) (layer "F.Cu") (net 10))
 (segment (start 165.8975 74.7675) (end 167.62 74.7675) (width 0.25) (layer "F.Cu") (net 10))
 (segment (start 151.0775 83.82) (end 151.13 83.82) (width 0.25) (layer "F.Cu") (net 10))
 (segment (start 135.929 101.5085) (end 135.9815 101.5085) (width 0.25) (layer "F.Cu") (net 9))
 (segment (start 134.8475 102.59) (end 135.929 101.5085) (width 0.25) (layer "F.Cu") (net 9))
 (segment (start 165.1 76.835) (end 165.5725 77.3075) (width 0.25) (layer "F.Cu") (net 9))
 (segment (start 161.925 72.39) (end 165.1 75.565) (width 0.25) (layer "F.Cu") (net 9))
 (segment (start 153.035 77.47) (end 158.115 72.39) (width 0.25) (layer "F.Cu") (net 9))
 (segment (start 135.9815 101.5085) (end 153.035 84.455) (width 0.25) (layer "F.Cu") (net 9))
 (segment (start 165.1 75.565) (end 165.1 76.835) (width 0.25) (layer "F.Cu") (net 9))
 (segment (start 158.115 72.39) (end 161.925 72.39) (width 0.25) (layer "F.Cu") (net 9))
 (segment (start 165.5725 77.3075) (end 167.62 77.3075) (width 0.25) (layer "F.Cu") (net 9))
 (segment (start 153.035 84.455) (end 153.035 77.47) (width 0.25) (layer "F.Cu") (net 9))
 (segment (start 158.75 81.28) (end 158.6975 81.28) (width 0.25) (layer "F.Cu") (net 20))
 (segment (start 158.789 81.241) (end 158.75 81.28) (width 0.25) (layer "F.Cu") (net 20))
 (segment (start 163.83 83.185) (end 161.886 81.241) (width 0.25) (layer "F.Cu") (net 20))
 (segment (start 167.62 89.3725) (end 166.55934 89.3725) (width 0.25) (layer "F.Cu") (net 20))
 (segment (start 163.83 86.64316) (end 163.83 83.185) (width 0.25) (layer "F.Cu") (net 20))
 (segment (start 161.886 81.241) (end 158.789 81.241) (width 0.25) (layer "F.Cu") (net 20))
 (segment (start 166.55934 89.3725) (end 163.83 86.64316) (width 0.25) (layer "F.Cu") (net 20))
 (segment (start 158.6975 81.28) (end 134.8475 105.13) (width 0.25) (layer "F.Cu") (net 20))
 (segment (start 170.16 89.58184) (end 170.16 90.6425) (width 0.25) (layer "F.Cu") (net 19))
 (segment (start 165.735 82.6775) (end 165.735 86.995) (width 0.25) (layer "F.Cu") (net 19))
 (segment (start 160.2475 77.19) (end 165.735 82.6775) (width 0.25) (layer "F.Cu") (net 19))
 (segment (start 165.735 86.995) (end 167.57316 86.995) (width 0.25) (layer "F.Cu") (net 19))
 (segment (start 167.57316 86.995) (end 170.16 89.58184) (width 0.25) (layer "F.Cu") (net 19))
 (segment (start 160.2475 82.27) (end 161.2765 83.299) (width 0.25) (layer "F.Cu") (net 18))
 (segment (start 161.2765 85.0765) (end 167.62 91.42) (width 0.25) (layer "F.Cu") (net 18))
 (segment (start 167.62 91.42) (end 167.62 91.9125) (width 0.25) (layer "F.Cu") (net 18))
 (segment (start 161.2765 83.299) (end 161.2765 85.0765) (width 0.25) (layer "F.Cu") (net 18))
 (segment (start 167.36972 93.1825) (end 170.16 93.1825) (width 0.25) (layer "F.Cu") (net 17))
 (segment (start 166.545 91.1075) (end 166.545 92.35778) (width 0.25) (layer "F.Cu") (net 17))
 (segment (start 160.2475 84.81) (end 166.545 91.1075) (width 0.25) (layer "F.Cu") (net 17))
 (segment (start 166.545 92.35778) (end 167.36972 93.1825) (width 0.25) (layer "F.Cu") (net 17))
 (segment (start 160.2475 92.43) (end 165.5975 92.43) (width 0.25) (layer "F.Cu") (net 16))
 (segment (start 165.5975 92.43) (end 167.62 94.4525) (width 0.25) (layer "F.Cu") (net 16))
 (segment (start 160.2475 94.97) (end 165.5975 94.97) (width 0.25) (layer "F.Cu") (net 15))
 (segment (start 165.5975 94.97) (end 167.62 96.9925) (width 0.25) (layer "F.Cu") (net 15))
 (segment (start 170.16 109.2) (end 170.16 110.3275) (width 0.25) (layer "F.Cu") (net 7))
 (segment (start 163.83 103.505) (end 167.64 107.315) (width 0.25) (layer "F.Cu") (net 7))
 (segment (start 167.64 107.315) (end 168.275 107.315) (width 0.25) (layer "F.Cu") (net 7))
 (segment (start 168.275 107.315) (end 170.16 109.2) (width 0.25) (layer "F.Cu") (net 7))
 (segment (start 163.83 101.0925) (end 163.83 103.505) (width 0.25) (layer "F.Cu") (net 7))
 (segment (start 160.2475 97.51) (end 163.83 101.0925) (width 0.25) (layer "F.Cu") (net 7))
 (segment (start 166.8425 109.0575) (end 162.56 104.775) (width 0.25) (layer "F.Cu") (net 8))
 (segment (start 162.56 104.775) (end 162.56 102.3625) (width 0.25) (layer "F.Cu") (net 8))
 (segment (start 167.62 109.0575) (end 166.8425 109.0575) (width 0.25) (layer "F.Cu") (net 8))
 (segment (start 162.56 102.3625) (end 160.2475 100.05) (width 0.25) (layer "F.Cu") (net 8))
 (segment (start 160.2475 102.59) (end 161.2765 103.619) (width 0.25) (layer "F.Cu") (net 6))
 (segment (start 161.2765 103.619) (end 161.2765 105.254) (width 0.25) (layer "F.Cu") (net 6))
 (segment (start 161.2765 105.254) (end 167.62 111.5975) (width 0.25) (layer "F.Cu") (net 6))
 (segment (start 160.2475 106.125606) (end 166.989394 112.8675) (width 0.25) (layer "F.Cu") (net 5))
 (segment (start 160.2475 105.13) (end 160.2475 106.125606) (width 0.25) (layer "F.Cu") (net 5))
 (segment (start 166.989394 112.8675) (end 170.16 112.8675) (width 0.25) (layer "F.Cu") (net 5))
 (segment (start 163.6925 110.21) (end 167.62 114.1375) (width 0.25) (layer "F.Cu") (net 4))
 (segment (start 160.2475 110.21) (end 163.6925 110.21) (width 0.25) (layer "F.Cu") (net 4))
 (segment (start 160.2475 112.75) (end 163.6925 112.75) (width 0.25) (layer "F.Cu") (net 2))
 (segment (start 163.6925 112.75) (end 167.62 116.6775) (width 0.25) (layer "F.Cu") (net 2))
 (segment (start 134.8475 120.37) (end 147.955 107.2625) (width 1) (layer "F.Cu") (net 31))
 (segment (start 147.955 107.2625) (end 147.955 95.25) (width 1) (layer "F.Cu") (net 31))
 (via (at 147.955 95.25) (size 0.8) (drill 0.4) (layers "F.Cu" "B.Cu") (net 31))
 (segment (start 147.955 95.25) (end 147.955 69.85) (width 1) (layer "B.Cu") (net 31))
 (segment (start 147.955 69.85) (end 161.29 56.515) (width 1) (layer "B.Cu") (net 31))
 (segment (start 161.29 56.515) (end 161.925 56.515) (width 1) (layer "B.Cu") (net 31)))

